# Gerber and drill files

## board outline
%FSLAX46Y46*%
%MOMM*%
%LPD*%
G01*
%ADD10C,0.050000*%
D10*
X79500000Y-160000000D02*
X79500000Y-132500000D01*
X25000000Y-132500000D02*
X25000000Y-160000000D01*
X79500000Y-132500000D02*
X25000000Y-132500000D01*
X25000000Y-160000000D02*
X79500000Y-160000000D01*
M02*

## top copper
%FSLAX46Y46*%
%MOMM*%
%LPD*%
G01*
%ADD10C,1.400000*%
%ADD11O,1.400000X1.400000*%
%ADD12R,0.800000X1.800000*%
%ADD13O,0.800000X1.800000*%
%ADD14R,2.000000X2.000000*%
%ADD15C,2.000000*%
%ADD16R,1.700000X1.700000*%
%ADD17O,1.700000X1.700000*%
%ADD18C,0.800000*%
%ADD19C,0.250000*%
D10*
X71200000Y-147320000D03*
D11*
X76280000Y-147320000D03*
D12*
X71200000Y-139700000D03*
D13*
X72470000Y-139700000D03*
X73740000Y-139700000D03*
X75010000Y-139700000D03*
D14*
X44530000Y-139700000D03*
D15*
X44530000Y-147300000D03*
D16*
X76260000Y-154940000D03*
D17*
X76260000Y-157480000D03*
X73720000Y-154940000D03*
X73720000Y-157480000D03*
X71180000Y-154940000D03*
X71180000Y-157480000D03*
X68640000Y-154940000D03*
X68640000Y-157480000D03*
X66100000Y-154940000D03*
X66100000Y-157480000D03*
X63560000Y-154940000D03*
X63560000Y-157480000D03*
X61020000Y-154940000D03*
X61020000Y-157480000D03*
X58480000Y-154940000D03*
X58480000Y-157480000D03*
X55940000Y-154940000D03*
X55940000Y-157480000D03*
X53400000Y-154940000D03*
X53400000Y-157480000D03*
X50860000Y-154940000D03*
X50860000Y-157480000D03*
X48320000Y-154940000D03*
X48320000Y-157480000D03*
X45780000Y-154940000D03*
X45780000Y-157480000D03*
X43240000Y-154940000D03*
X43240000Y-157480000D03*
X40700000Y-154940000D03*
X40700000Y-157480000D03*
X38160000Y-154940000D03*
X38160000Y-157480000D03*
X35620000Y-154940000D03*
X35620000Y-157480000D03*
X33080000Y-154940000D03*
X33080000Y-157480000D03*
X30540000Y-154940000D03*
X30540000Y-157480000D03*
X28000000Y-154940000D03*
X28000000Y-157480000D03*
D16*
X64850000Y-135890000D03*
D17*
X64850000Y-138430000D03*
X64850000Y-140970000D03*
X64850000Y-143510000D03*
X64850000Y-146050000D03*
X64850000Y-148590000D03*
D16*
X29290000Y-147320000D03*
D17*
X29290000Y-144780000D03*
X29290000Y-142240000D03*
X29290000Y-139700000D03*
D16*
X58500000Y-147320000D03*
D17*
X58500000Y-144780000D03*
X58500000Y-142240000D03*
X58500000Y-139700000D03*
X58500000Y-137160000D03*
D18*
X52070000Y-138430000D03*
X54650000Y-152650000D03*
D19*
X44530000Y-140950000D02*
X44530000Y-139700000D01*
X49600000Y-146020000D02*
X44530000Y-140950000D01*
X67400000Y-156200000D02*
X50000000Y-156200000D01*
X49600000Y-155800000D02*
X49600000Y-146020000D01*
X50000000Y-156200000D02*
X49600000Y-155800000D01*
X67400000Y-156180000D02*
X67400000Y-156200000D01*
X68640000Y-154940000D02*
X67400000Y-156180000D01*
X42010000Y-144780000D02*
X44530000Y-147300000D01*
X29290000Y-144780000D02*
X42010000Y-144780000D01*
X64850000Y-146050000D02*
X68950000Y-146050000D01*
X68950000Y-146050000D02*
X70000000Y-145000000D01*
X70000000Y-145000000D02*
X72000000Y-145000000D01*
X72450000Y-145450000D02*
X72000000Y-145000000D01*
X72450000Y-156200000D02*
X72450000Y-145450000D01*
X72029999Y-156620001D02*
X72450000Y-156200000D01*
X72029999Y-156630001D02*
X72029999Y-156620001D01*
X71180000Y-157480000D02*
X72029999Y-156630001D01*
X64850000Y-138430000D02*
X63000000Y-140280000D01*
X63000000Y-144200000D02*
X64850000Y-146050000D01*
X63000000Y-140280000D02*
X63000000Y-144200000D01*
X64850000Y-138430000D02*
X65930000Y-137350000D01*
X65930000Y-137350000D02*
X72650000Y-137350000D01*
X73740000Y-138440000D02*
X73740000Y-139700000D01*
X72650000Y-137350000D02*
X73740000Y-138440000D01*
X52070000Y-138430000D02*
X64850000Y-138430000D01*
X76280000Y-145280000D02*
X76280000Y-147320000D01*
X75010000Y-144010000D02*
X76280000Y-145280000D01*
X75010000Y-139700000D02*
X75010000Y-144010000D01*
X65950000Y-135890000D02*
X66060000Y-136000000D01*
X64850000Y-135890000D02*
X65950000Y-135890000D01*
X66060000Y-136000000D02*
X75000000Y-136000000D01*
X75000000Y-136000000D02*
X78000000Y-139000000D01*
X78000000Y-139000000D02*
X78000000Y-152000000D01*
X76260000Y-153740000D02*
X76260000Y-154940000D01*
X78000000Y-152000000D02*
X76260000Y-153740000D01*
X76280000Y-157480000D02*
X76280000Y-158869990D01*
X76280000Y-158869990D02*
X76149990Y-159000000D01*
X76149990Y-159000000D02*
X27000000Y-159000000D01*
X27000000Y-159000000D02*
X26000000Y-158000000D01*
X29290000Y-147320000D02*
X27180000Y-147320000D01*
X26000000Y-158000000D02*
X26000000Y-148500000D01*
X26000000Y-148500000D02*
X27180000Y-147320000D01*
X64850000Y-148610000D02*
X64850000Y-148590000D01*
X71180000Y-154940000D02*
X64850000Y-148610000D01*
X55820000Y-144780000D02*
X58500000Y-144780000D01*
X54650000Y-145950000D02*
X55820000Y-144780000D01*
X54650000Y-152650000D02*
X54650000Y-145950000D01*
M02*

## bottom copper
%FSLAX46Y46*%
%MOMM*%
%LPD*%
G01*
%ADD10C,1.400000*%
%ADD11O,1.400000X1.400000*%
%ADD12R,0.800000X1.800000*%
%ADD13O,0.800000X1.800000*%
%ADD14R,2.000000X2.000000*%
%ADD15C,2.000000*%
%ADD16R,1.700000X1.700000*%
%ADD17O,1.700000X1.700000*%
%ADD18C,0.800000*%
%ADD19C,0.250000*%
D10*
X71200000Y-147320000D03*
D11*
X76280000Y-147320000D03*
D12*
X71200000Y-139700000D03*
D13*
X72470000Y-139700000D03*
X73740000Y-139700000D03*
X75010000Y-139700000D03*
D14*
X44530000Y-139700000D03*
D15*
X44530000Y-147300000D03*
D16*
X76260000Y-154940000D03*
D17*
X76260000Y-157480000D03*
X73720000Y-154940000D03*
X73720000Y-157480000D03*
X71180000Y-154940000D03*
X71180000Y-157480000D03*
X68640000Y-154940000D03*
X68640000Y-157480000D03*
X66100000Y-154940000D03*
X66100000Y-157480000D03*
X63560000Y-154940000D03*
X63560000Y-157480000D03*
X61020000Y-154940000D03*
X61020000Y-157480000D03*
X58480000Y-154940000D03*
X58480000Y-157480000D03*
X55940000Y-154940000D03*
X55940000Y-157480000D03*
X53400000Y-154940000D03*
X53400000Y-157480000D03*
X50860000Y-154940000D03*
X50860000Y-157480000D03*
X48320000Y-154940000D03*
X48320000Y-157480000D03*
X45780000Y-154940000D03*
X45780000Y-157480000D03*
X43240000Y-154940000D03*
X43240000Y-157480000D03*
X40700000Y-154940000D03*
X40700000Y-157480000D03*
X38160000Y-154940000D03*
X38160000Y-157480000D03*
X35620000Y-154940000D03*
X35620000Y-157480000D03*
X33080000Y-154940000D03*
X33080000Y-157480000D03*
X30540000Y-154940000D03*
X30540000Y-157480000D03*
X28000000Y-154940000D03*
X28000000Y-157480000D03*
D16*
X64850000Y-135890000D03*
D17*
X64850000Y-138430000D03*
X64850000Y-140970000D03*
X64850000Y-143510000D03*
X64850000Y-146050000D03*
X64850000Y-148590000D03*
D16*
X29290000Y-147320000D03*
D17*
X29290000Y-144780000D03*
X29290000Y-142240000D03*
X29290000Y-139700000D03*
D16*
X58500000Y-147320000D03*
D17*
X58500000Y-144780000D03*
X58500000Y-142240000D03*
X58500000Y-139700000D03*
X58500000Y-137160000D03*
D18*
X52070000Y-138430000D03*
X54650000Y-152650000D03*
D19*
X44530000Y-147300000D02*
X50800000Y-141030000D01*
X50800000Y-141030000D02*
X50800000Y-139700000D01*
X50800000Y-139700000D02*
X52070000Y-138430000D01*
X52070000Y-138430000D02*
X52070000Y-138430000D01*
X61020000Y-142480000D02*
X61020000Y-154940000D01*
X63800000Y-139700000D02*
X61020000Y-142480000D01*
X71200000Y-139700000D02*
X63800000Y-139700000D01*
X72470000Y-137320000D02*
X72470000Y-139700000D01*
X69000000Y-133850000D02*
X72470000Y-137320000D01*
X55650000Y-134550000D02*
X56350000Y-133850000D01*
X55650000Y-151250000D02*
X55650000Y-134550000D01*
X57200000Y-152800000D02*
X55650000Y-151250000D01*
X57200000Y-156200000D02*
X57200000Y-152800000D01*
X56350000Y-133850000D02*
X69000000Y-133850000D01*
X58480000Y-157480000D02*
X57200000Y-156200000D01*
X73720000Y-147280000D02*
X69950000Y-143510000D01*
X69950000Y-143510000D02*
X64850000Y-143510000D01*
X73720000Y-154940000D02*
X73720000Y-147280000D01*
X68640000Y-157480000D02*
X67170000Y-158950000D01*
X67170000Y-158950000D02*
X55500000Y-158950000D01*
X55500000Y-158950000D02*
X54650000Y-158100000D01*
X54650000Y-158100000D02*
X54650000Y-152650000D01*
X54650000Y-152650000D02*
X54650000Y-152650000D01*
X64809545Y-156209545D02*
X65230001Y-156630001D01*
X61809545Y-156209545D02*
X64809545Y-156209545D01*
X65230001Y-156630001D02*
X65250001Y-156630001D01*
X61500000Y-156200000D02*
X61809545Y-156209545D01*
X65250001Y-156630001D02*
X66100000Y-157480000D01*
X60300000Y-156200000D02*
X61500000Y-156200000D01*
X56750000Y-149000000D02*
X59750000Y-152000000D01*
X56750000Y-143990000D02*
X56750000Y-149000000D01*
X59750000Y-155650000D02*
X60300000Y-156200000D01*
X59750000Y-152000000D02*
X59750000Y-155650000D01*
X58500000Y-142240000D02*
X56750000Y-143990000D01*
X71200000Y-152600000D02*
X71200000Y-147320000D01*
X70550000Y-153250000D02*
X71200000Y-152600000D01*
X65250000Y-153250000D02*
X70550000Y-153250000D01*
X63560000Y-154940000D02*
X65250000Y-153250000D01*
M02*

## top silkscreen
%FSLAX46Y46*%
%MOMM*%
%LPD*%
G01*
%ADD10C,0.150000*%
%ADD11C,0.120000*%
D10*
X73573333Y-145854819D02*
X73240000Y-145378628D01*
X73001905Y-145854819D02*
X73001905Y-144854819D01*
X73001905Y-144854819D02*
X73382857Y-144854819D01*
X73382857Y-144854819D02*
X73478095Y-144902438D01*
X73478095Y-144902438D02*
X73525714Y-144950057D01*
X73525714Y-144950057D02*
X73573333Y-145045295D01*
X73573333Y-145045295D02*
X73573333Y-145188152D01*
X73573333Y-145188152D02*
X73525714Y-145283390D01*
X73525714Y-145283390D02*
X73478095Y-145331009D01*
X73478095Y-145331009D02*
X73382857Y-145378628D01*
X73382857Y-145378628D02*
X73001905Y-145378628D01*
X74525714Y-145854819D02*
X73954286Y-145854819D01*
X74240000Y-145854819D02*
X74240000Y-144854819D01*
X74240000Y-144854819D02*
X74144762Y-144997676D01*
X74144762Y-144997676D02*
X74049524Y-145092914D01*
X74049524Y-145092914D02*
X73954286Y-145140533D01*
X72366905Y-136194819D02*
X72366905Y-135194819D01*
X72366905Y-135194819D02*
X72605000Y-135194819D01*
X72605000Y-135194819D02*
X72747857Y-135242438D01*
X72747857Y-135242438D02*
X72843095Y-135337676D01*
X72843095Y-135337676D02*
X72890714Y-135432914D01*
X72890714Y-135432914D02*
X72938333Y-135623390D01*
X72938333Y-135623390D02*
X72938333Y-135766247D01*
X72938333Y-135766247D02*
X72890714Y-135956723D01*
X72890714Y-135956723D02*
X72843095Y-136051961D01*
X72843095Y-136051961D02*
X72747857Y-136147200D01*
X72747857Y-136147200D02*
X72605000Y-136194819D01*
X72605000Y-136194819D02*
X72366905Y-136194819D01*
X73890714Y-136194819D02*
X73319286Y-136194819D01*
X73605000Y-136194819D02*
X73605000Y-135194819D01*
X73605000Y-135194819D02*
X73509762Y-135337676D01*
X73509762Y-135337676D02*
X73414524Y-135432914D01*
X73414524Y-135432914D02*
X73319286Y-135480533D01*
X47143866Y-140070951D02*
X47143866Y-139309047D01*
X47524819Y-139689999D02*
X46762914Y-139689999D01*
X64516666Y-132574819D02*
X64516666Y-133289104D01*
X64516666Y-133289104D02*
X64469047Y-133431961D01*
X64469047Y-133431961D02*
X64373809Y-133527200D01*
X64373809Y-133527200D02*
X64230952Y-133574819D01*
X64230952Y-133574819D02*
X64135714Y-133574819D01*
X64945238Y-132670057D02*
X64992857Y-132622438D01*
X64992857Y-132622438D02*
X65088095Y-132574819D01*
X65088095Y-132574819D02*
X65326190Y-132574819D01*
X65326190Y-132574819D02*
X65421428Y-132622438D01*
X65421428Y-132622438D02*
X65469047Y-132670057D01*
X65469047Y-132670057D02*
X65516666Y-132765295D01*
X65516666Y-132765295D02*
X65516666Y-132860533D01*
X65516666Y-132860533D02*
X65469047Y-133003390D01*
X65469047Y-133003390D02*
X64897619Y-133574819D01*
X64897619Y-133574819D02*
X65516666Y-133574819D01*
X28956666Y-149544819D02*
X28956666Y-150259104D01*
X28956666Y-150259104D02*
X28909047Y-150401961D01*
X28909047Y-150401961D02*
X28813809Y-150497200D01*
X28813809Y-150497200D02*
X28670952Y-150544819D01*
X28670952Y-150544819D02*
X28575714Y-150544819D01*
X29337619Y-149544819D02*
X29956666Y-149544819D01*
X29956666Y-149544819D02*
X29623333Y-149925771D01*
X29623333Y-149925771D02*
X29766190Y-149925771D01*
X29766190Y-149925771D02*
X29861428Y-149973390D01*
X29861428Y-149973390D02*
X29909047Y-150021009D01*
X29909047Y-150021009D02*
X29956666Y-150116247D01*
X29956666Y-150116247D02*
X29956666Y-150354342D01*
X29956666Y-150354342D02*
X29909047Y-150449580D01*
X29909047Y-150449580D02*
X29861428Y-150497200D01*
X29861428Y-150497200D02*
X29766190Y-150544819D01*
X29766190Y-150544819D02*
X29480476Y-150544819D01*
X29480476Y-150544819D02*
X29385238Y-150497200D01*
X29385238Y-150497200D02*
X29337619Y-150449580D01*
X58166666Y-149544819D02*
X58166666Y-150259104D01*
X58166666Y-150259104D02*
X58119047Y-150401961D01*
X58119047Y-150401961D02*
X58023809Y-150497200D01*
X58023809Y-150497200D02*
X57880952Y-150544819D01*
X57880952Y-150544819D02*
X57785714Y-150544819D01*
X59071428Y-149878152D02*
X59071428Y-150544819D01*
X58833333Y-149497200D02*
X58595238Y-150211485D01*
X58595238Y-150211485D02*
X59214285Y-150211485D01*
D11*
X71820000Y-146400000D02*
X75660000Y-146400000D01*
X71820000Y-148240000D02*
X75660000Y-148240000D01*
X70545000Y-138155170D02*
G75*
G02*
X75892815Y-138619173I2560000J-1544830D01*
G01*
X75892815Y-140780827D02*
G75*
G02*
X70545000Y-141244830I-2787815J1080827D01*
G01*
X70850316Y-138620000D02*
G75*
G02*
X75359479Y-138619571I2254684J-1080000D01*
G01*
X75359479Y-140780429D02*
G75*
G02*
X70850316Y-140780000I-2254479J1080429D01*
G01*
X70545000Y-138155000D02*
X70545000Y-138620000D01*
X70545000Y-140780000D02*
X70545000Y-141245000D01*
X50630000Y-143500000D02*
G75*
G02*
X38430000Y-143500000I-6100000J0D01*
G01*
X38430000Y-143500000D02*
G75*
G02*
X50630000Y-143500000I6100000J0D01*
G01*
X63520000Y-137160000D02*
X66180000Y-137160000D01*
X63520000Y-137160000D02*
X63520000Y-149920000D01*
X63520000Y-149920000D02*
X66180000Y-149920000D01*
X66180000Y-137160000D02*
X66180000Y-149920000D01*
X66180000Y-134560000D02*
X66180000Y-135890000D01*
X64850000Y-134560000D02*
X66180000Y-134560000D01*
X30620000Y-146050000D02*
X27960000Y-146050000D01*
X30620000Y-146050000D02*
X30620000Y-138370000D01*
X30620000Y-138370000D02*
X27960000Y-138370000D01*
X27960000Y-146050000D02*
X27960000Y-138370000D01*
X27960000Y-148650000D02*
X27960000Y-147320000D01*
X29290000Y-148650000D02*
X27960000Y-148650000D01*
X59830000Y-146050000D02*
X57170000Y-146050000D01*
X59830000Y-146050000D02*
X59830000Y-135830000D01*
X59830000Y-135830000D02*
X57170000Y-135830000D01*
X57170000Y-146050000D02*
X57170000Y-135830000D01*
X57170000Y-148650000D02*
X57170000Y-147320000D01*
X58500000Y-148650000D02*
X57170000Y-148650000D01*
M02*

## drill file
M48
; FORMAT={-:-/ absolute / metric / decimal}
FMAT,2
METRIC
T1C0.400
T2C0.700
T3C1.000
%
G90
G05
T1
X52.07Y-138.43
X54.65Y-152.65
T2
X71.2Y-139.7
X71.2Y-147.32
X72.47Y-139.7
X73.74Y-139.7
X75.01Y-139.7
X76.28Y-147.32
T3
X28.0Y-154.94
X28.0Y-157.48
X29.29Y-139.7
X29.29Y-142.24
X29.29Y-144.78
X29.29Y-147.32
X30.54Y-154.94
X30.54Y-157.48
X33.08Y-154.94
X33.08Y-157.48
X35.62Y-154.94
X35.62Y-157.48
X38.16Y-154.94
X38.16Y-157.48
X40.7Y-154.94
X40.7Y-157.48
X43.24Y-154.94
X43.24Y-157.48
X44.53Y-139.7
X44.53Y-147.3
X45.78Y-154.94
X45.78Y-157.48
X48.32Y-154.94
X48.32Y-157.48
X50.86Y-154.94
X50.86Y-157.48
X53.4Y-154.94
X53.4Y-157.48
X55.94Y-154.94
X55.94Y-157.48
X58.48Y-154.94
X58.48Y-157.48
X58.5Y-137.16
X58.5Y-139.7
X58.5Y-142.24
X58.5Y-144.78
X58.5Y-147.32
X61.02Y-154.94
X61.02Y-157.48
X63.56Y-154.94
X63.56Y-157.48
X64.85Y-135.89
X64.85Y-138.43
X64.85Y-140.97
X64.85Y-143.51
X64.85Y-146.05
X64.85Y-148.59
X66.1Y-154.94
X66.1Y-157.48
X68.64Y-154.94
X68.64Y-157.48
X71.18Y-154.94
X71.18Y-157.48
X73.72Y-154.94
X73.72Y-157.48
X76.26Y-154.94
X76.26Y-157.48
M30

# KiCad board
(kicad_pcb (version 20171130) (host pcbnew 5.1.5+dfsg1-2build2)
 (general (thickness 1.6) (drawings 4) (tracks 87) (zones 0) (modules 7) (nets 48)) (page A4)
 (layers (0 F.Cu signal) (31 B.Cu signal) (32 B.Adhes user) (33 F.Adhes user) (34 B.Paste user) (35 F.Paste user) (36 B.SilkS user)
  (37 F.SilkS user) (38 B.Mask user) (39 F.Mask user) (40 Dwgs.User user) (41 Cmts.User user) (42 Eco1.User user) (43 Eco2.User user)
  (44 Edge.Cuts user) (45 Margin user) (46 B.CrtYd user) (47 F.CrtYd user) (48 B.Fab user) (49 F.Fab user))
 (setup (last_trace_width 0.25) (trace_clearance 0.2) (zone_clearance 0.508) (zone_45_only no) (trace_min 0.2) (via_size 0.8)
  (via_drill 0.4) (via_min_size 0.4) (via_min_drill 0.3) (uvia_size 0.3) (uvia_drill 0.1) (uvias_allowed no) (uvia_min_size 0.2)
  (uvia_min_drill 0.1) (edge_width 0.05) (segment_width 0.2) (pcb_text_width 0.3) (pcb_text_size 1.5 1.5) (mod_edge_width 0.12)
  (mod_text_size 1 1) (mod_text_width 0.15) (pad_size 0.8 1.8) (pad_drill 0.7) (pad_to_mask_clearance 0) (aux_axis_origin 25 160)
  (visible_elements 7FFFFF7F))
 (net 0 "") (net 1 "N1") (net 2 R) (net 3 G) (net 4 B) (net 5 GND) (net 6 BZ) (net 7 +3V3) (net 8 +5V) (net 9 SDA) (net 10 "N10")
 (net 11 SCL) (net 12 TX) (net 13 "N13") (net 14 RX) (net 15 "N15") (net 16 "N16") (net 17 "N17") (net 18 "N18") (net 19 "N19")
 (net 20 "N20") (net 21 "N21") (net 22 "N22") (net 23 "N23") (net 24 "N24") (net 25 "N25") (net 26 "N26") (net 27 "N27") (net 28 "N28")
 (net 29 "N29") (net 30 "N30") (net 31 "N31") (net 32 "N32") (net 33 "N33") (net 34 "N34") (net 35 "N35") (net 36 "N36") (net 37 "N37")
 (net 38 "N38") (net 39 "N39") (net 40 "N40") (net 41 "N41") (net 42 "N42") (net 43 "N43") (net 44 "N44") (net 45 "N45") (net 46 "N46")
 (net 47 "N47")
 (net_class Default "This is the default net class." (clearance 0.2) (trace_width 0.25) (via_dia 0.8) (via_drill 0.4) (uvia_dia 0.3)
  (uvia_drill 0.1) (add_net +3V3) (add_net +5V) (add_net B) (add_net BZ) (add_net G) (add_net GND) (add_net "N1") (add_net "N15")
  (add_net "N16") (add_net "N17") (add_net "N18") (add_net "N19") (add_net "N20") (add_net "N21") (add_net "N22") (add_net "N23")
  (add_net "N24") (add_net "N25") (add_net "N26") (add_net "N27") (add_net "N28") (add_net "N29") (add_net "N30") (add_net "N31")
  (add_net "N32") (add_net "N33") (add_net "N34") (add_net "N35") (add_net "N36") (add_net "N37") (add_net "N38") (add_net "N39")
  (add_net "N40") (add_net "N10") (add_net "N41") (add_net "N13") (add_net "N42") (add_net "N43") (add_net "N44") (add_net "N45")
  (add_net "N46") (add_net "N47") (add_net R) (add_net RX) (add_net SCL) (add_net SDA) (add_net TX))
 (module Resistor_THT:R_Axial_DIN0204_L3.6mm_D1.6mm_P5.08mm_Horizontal (layer F.Cu) (at 71.2 147.32)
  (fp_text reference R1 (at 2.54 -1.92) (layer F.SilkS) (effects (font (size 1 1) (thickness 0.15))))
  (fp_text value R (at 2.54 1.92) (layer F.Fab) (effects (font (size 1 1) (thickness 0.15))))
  (fp_line (start 0.62 -0.92) (end 4.46 -0.92) (layer F.SilkS) (width 0.12))
  (fp_line (start 0.62 0.92) (end 4.46 0.92) (layer F.SilkS) (width 0.12))
  (pad 1 thru_hole circle (at 0 0) (size 1.4 1.4) (drill 0.7) (layers *.Cu *.Mask) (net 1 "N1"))
  (pad 2 thru_hole oval (at 5.08 0) (size 1.4 1.4) (drill 0.7) (layers *.Cu *.Mask) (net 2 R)))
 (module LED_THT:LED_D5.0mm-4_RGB (layer F.Cu) (at 71.2 139.7)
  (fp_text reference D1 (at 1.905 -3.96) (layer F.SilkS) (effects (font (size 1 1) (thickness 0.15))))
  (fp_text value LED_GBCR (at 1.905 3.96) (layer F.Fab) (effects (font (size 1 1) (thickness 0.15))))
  (fp_arc (start 1.905 0) (end -0.655 -1.54483) (angle 127.7) (layer F.SilkS) (width 0.12))
  (fp_arc (start 1.905 0) (end -0.655 1.54483) (angle -127.7) (layer F.SilkS) (width 0.12))
  (fp_arc (start 1.905 0) (end -0.349684 -1.08) (angle 128.8) (layer F.SilkS) (width 0.12))
  (fp_arc (start 1.905 0) (end -0.349684 1.08) (angle -128.8) (layer F.SilkS) (width 0.12))
  (fp_line (start -0.655 -1.545) (end -0.655 -1.08) (layer F.SilkS) (width 0.12))
  (fp_line (start -0.655 1.08) (end -0.655 1.545) (layer F.SilkS) (width 0.12))
  (pad 1 thru_hole rect (at 0 0) (size 0.8 1.8) (drill 0.7) (layers *.Cu *.Mask) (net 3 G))
  (pad 2 thru_hole oval (at 1.27 0) (size 0.8 1.8) (drill 0.7) (layers *.Cu *.Mask) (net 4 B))
  (pad 3 thru_hole oval (at 2.54 0) (size 0.8 1.8) (drill 0.7) (layers *.Cu *.Mask) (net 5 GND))
  (pad 4 thru_hole oval (at 3.81 0) (size 0.8 1.8) (drill 0.7) (layers *.Cu *.Mask) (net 2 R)))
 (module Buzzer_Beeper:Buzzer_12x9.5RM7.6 (layer F.Cu) (at 44.53 139.7 270)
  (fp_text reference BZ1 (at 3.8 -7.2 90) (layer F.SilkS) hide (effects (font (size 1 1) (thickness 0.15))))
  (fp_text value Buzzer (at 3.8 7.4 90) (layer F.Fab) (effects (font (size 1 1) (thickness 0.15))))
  (fp_circle (center 3.8 0) (end 9.9 0) (layer F.SilkS) (width 0.12))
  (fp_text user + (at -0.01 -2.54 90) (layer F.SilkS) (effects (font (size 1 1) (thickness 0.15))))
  (pad 1 thru_hole rect (at 0 0 270) (size 2 2) (drill 1) (layers *.Cu *.Mask) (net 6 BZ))
  (pad 2 thru_hole circle (at 7.6 0 270) (size 2 2) (drill 1) (layers *.Cu *.Mask) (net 5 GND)))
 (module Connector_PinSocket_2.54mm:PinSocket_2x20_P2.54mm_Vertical (layer B.Cu) (at 76.26 154.94 90)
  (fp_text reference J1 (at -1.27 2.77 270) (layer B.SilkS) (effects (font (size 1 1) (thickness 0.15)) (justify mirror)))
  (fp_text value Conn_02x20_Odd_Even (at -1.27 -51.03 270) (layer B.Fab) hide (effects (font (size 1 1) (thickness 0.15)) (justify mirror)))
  (pad 1 thru_hole rect (at 0 0 90) (size 1.7 1.7) (drill 1) (layers *.Cu *.Mask) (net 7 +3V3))
  (pad 2 thru_hole oval (at -2.54 0 90) (size 1.7 1.7) (drill 1) (layers *.Cu *.Mask) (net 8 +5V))
  (pad 3 thru_hole oval (at 0 -2.54 90) (size 1.7 1.7) (drill 1) (layers *.Cu *.Mask) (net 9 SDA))
  (pad 4 thru_hole oval (at -2.54 -2.54 90) (size 1.7 1.7) (drill 1) (layers *.Cu *.Mask) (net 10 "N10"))
  (pad 5 thru_hole oval (at 0 -5.08 90) (size 1.7 1.7) (drill 1) (layers *.Cu *.Mask) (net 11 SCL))
  (pad 6 thru_hole oval (at -2.54 -5.08 90) (size 1.7 1.7) (drill 1) (layers *.Cu *.Mask) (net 5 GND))
  (pad 7 thru_hole oval (at 0 -7.62 90) (size 1.7 1.7) (drill 1) (layers *.Cu *.Mask) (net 6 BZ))
  (pad 8 thru_hole oval (at -2.54 -7.62 90) (size 1.7 1.7) (drill 1) (layers *.Cu *.Mask) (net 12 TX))
  (pad 9 thru_hole oval (at 0 -10.16 90) (size 1.7 1.7) (drill 1) (layers *.Cu *.Mask) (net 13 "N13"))
  (pad 10 thru_hole oval (at -2.54 -10.16 90) (size 1.7 1.7) (drill 1) (layers *.Cu *.Mask) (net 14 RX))
  (pad 11 thru_hole oval (at 0 -12.7 90) (size 1.7 1.7) (drill 1) (layers *.Cu *.Mask) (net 1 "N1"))
  (pad 12 thru_hole oval (at -2.54 -12.7 90) (size 1.7 1.7) (drill 1) (layers *.Cu *.Mask) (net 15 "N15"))
  (pad 13 thru_hole oval (at 0 -15.24 90) (size 1.7 1.7) (drill 1) (layers *.Cu *.Mask) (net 3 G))
  (pad 14 thru_hole oval (at -2.54 -15.24 90) (size 1.7 1.7) (drill 1) (layers *.Cu *.Mask) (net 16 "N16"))
  (pad 15 thru_hole oval (at 0 -17.78 90) (size 1.7 1.7) (drill 1) (layers *.Cu *.Mask) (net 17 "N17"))
  (pad 16 thru_hole oval (at -2.54 -17.78 90) (size 1.7 1.7) (drill 1) (layers *.Cu *.Mask) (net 4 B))
  (pad 17 thru_hole oval (at 0 -20.32 90) (size 1.7 1.7) (drill 1) (layers *.Cu *.Mask) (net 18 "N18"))
  (pad 18 thru_hole oval (at -2.54 -20.32 90) (size 1.7 1.7) (drill 1) (layers *.Cu *.Mask) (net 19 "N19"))
  (pad 19 thru_hole oval (at 0 -22.86 90) (size 1.7 1.7) (drill 1) (layers *.Cu *.Mask) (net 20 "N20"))
  (pad 20 thru_hole oval (at -2.54 -22.86 90) (size 1.7 1.7) (drill 1) (layers *.Cu *.Mask) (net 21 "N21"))
  (pad 21 thru_hole oval (at 0 -25.4 90) (size 1.7 1.7) (drill 1) (layers *.Cu *.Mask) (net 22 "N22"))
  (pad 22 thru_hole oval (at -2.54 -25.4 90) (size 1.7 1.7) (drill 1) (layers *.Cu *.Mask) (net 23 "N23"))
  (pad 23 thru_hole oval (at 0 -27.94 90) (size 1.7 1.7) (drill 1) (layers *.Cu *.Mask) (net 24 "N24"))
  (pad 24 thru_hole oval (at -2.54 -27.94 90) (size 1.7 1.7) (drill 1) (layers *.Cu *.Mask) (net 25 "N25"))
  (pad 25 thru_hole oval (at 0 -30.48 90) (size 1.7 1.7) (drill 1) (layers *.Cu *.Mask) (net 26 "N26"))
  (pad 26 thru_hole oval (at -2.54 -30.48 90) (size 1.7 1.7) (drill 1) (layers *.Cu *.Mask) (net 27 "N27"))
  (pad 27 thru_hole oval (at 0 -33.02 90) (size 1.7 1.7) (drill 1) (layers *.Cu *.Mask) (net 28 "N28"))
  (pad 28 thru_hole oval (at -2.54 -33.02 90) (size 1.7 1.7) (drill 1) (layers *.Cu *.Mask) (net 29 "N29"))
  (pad 29 thru_hole oval (at 0 -35.56 90) (size 1.7 1.7) (drill 1) (layers *.Cu *.Mask) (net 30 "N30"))
  (pad 30 thru_hole oval (at -2.54 -35.56 90) (size 1.7 1.7) (drill 1) (layers *.Cu *.Mask) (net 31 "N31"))
  (pad 31 thru_hole oval (at 0 -38.1 90) (size 1.7 1.7) (drill 1) (layers *.Cu *.Mask) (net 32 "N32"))
  (pad 32 thru_hole oval (at -2.54 -38.1 90) (size 1.7 1.7) (drill 1) (layers *.Cu *.Mask) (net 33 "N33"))
  (pad 33 thru_hole oval (at 0 -40.64 90) (size 1.7 1.7) (drill 1) (layers *.Cu *.Mask) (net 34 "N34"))
  (pad 34 thru_hole oval (at -2.54 -40.64 90) (size 1.7 1.7) (drill 1) (layers *.Cu *.Mask) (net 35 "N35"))
  (pad 35 thru_hole oval (at 0 -43.18 90) (size 1.7 1.7) (drill 1) (layers *.Cu *.Mask) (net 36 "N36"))
  (pad 36 thru_hole oval (at -2.54 -43.18 90) (size 1.7 1.7) (drill 1) (layers *.Cu *.Mask) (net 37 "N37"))
  (pad 37 thru_hole oval (at 0 -45.72 90) (size 1.7 1.7) (drill 1) (layers *.Cu *.Mask) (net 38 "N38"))
  (pad 38 thru_hole oval (at -2.54 -45.72 90) (size 1.7 1.7) (drill 1) (layers *.Cu *.Mask) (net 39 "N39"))
  (pad 39 thru_hole oval (at 0 -48.26 90) (size 1.7 1.7) (drill 1) (layers *.Cu *.Mask) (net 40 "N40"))
  (pad 40 thru_hole oval (at -2.54 -48.26 90) (size 1.7 1.7) (drill 1) (layers *.Cu *.Mask) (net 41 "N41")))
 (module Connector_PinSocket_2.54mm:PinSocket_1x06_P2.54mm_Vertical (layer F.Cu) (at 64.85 135.89)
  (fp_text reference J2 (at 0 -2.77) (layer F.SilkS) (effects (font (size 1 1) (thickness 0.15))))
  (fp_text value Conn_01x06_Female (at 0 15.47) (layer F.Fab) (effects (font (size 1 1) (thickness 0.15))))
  (fp_line (start -1.33 1.27) (end 1.33 1.27) (layer F.SilkS) (width 0.12))
  (fp_line (start -1.33 1.27) (end -1.33 14.03) (layer F.SilkS) (width 0.12))
  (fp_line (start -1.33 14.03) (end 1.33 14.03) (layer F.SilkS) (width 0.12))
  (fp_line (start 1.33 1.27) (end 1.33 14.03) (layer F.SilkS) (width 0.12))
  (fp_line (start 1.33 -1.33) (end 1.33 0) (layer F.SilkS) (width 0.12))
  (fp_line (start 0 -1.33) (end 1.33 -1.33) (layer F.SilkS) (width 0.12))
  (pad 1 thru_hole rect (at 0 0) (size 1.7 1.7) (drill 1) (layers *.Cu *.Mask) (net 7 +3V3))
  (pad 2 thru_hole oval (at 0 2.54) (size 1.7 1.7) (drill 1) (layers *.Cu *.Mask) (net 5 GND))
  (pad 3 thru_hole oval (at 0 5.08) (size 1.7 1.7) (drill 1) (layers *.Cu *.Mask) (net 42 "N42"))
  (pad 4 thru_hole oval (at 0 7.62) (size 1.7 1.7) (drill 1) (layers *.Cu *.Mask) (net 9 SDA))
  (pad 5 thru_hole oval (at 0 10.16) (size 1.7 1.7) (drill 1) (layers *.Cu *.Mask) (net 5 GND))
  (pad 6 thru_hole oval (at 0 12.7) (size 1.7 1.7) (drill 1) (layers *.Cu *.Mask) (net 11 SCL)))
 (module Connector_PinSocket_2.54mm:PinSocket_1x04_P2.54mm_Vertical (layer F.Cu) (at 29.29 147.32 180)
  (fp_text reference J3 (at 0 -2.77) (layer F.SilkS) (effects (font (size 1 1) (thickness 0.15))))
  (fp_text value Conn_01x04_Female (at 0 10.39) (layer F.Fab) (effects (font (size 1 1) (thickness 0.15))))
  (fp_line (start -1.33 1.27) (end 1.33 1.27) (layer F.SilkS) (width 0.12))
  (fp_line (start -1.33 1.27) (end -1.33 8.95) (layer F.SilkS) (width 0.12))
  (fp_line (start -1.33 8.95) (end 1.33 8.95) (layer F.SilkS) (width 0.12))
  (fp_line (start 1.33 1.27) (end 1.33 8.95) (layer F.SilkS) (width 0.12))
  (fp_line (start 1.33 -1.33) (end 1.33 0) (layer F.SilkS) (width 0.12))
  (fp_line (start 0 -1.33) (end 1.33 -1.33) (layer F.SilkS) (width 0.12))
  (pad 1 thru_hole rect (at 0 0 180) (size 1.7 1.7) (drill 1) (layers *.Cu *.Mask) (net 8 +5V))
  (pad 2 thru_hole oval (at 0 2.54 180) (size 1.7 1.7) (drill 1) (layers *.Cu *.Mask) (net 5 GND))
  (pad 3 thru_hole oval (at 0 5.08 180) (size 1.7 1.7) (drill 1) (layers *.Cu *.Mask) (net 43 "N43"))
  (pad 4 thru_hole oval (at 0 7.62 180) (size 1.7 1.7) (drill 1) (layers *.Cu *.Mask) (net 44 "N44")))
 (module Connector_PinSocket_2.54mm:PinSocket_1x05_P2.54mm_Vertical (layer F.Cu) (at 58.5 147.32 180)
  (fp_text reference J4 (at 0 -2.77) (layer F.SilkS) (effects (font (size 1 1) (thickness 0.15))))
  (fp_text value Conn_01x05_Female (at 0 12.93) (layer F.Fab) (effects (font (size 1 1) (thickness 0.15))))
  (fp_line (start -1.33 1.27) (end 1.33 1.27) (layer F.SilkS) (width 0.12))
  (fp_line (start -1.33 1.27) (end -1.33 11.49) (layer F.SilkS) (width 0.12))
  (fp_line (start -1.33 11.49) (end 1.33 11.49) (layer F.SilkS) (width 0.12))
  (fp_line (start 1.33 1.27) (end 1.33 11.49) (layer F.SilkS) (width 0.12))
  (fp_line (start 1.33 -1.33) (end 1.33 0) (layer F.SilkS) (width 0.12))
  (fp_line (start 0 -1.33) (end 1.33 -1.33) (layer F.SilkS) (width 0.12))
  (pad 1 thru_hole rect (at 0 0 180) (size 1.7 1.7) (drill 1) (layers *.Cu *.Mask) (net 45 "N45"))
  (pad 2 thru_hole oval (at 0 2.54 180) (size 1.7 1.7) (drill 1) (layers *.Cu *.Mask) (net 12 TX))
  (pad 3 thru_hole oval (at 0 5.08 180) (size 1.7 1.7) (drill 1) (layers *.Cu *.Mask) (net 14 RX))
  (pad 4 thru_hole oval (at 0 7.62 180) (size 1.7 1.7) (drill 1) (layers *.Cu *.Mask) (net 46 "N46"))
  (pad 5 thru_hole oval (at 0 10.16 180) (size 1.7 1.7) (drill 1) (layers *.Cu *.Mask) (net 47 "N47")))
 (gr_line (start 79.5 160) (end 79.5 132.5) (layer Edge.Cuts) (width 0.05))
 (gr_line (start 25 132.5) (end 25 160) (layer Edge.Cuts) (width 0.05))
 (gr_line (start 79.5 132.5) (end 25 132.5) (layer Edge.Cuts) (width 0.05))
 (gr_line (start 25 160) (end 79.5 160) (layer Edge.Cuts) (width 0.05))
 (segment (start 44.53 140.95) (end 44.53 139.7) (width 0.25) (layer F.Cu) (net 6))
 (segment (start 49.6 146.02) (end 44.53 140.95) (width 0.25) (layer F.Cu) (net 6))
 (segment (start 67.4 156.2) (end 50 156.2) (width 0.25) (layer F.Cu) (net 6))
 (segment (start 49.6 155.8) (end 49.6 146.02) (width 0.25) (layer F.Cu) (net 6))
 (segment (start 50 156.2) (end 49.6 155.8) (width 0.25) (layer F.Cu) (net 6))
 (segment (start 67.4 156.18) (end 67.4 156.2) (width 0.25) (layer F.Cu) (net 6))
 (segment (start 68.64 154.94) (end 67.4 156.18) (width 0.25) (layer F.Cu) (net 6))
 (segment (start 42.01 144.78) (end 44.53 147.3) (width 0.25) (layer F.Cu) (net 5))
 (segment (start 29.29 144.78) (end 42.01 144.78) (width 0.25) (layer F.Cu) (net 5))
 (segment (start 64.85 146.05) (end 68.95 146.05) (width 0.25) (layer F.Cu) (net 5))
 (segment (start 68.95 146.05) (end 70 145) (width 0.25) (layer F.Cu) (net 5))
 (segment (start 70 145) (end 72 145) (width 0.25) (layer F.Cu) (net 5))
 (segment (start 72.45 145.45) (end 72 145) (width 0.25) (layer F.Cu) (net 5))
 (segment (start 72.45 156.2) (end 72.45 145.45) (width 0.25) (layer F.Cu) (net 5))
 (segment (start 72.029999 156.620001) (end 72.45 156.2) (width 0.25) (layer F.Cu) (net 5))
 (segment (start 72.029999 156.630001) (end 72.029999 156.620001) (width 0.25) (layer F.Cu) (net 5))
 (segment (start 71.18 157.48) (end 72.029999 156.630001) (width 0.25) (layer F.Cu) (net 5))
 (segment (start 64.85 138.43) (end 63 140.28) (width 0.25) (layer F.Cu) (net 5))
 (segment (start 63 144.2) (end 64.85 146.05) (width 0.25) (layer F.Cu) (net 5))
 (segment (start 63 140.28) (end 63 144.2) (width 0.25) (layer F.Cu) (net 5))
 (segment (start 64.85 138.43) (end 65.93 137.35) (width 0.25) (layer F.Cu) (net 5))
 (segment (start 65.93 137.35) (end 72.65 137.35) (width 0.25) (layer F.Cu) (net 5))
 (segment (start 73.74 138.44) (end 73.74 139.7) (width 0.25) (layer F.Cu) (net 5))
 (segment (start 72.65 137.35) (end 73.74 138.44) (width 0.25) (layer F.Cu) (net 5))
 (segment (start 44.53 147.3) (end 50.8 141.03) (width 0.25) (layer B.Cu) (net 5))
 (segment (start 50.8 141.03) (end 50.8 139.7) (width 0.25) (layer B.Cu) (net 5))
 (segment (start 50.8 139.7) (end 52.07 138.43) (width 0.25) (layer B.Cu) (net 5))
 (segment (start 52.07 138.43) (end 52.07 138.43) (width 0.25) (layer B.Cu) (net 5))
 (via (at 52.07 138.43) (size 0.8) (drill 0.4) (layers F.Cu B.Cu) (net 5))
 (segment (start 52.07 138.43) (end 64.85 138.43) (width 0.25) (layer F.Cu) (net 5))
 (segment (start 61.02 142.48) (end 61.02 154.94) (width 0.25) (layer B.Cu) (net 3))
 (segment (start 63.8 139.7) (end 61.02 142.48) (width 0.25) (layer B.Cu) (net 3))
 (segment (start 71.2 139.7) (end 63.8 139.7) (width 0.25) (layer B.Cu) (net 3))
 (segment (start 72.47 137.32) (end 72.47 139.7) (width 0.25) (layer B.Cu) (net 4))
 (segment (start 69 133.85) (end 72.47 137.32) (width 0.25) (layer B.Cu) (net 4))
 (segment (start 55.65 134.55) (end 56.35 133.85) (width 0.25) (layer B.Cu) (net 4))
 (segment (start 55.65 151.25) (end 55.65 134.55) (width 0.25) (layer B.Cu) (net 4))
 (segment (start 57.2 152.8) (end 55.65 151.25) (width 0.25) (layer B.Cu) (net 4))
 (segment (start 57.2 156.2) (end 57.2 152.8) (width 0.25) (layer B.Cu) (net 4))
 (segment (start 56.35 133.85) (end 69 133.85) (width 0.25) (layer B.Cu) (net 4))
 (segment (start 58.48 157.48) (end 57.2 156.2) (width 0.25) (layer B.Cu) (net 4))
 (segment (start 76.28 145.28) (end 76.28 147.32) (width 0.25) (layer F.Cu) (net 2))
 (segment (start 75.01 144.01) (end 76.28 145.28) (width 0.25) (layer F.Cu) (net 2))
 (segment (start 75.01 139.7) (end 75.01 144.01) (width 0.25) (layer F.Cu) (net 2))
 (segment (start 65.95 135.89) (end 66.06 136) (width 0.25) (layer F.Cu) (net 7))
 (segment (start 64.85 135.89) (end 65.95 135.89) (width 0.25) (layer F.Cu) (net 7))
 (segment (start 66.06 136) (end 75 136) (width 0.25) (layer F.Cu) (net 7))
 (segment (start 75 136) (end 78 139) (width 0.25) (layer F.Cu) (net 7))
 (segment (start 78 139) (end 78 152) (width 0.25) (layer F.Cu) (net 7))
 (segment (start 76.26 153.74) (end 76.26 154.94) (width 0.25) (layer F.Cu) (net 7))
 (segment (start 78 152) (end 76.26 153.74) (width 0.25) (layer F.Cu) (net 7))
 (segment (start 76.28 157.48) (end 76.28 158.86999) (width 0.25) (layer F.Cu) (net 8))
 (segment (start 76.28 158.86999) (end 76.14999 159) (width 0.25) (layer F.Cu) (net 8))
 (segment (start 76.14999 159) (end 27 159) (width 0.25) (layer F.Cu) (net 8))
 (segment (start 27 159) (end 26 158) (width 0.25) (layer F.Cu) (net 8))
 (segment (start 29.29 147.32) (end 27.18 147.32) (width 0.25) (layer F.Cu) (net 8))
 (segment (start 26 158) (end 26 148.5) (width 0.25) (layer F.Cu) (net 8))
 (segment (start 26 148.5) (end 27.18 147.32) (width 0.25) (layer F.Cu) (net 8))
 (segment (start 73.72 147.28) (end 69.95 143.51) (width 0.25) (layer B.Cu) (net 9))
 (segment (start 69.95 143.51) (end 64.85 143.51) (width 0.25) (layer B.Cu) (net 9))
 (segment (start 73.72 154.94) (end 73.72 147.28) (width 0.25) (layer B.Cu) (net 9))
 (segment (start 64.85 148.61) (end 64.85 148.59) (width 0.25) (layer F.Cu) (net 11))
 (segment (start 71.18 154.94) (end 64.85 148.61) (width 0.25) (layer F.Cu) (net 11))
 (segment (start 68.64 157.48) (end 67.17 158.95) (width 0.25) (layer B.Cu) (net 12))
 (segment (start 67.17 158.95) (end 55.5 158.95) (width 0.25) (layer B.Cu) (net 12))
 (segment (start 55.5 158.95) (end 54.65 158.1) (width 0.25) (layer B.Cu) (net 12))
 (segment (start 54.65 158.1) (end 54.65 152.65) (width 0.25) (layer B.Cu) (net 12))
 (segment (start 54.65 152.65) (end 54.65 152.65) (width 0.25) (layer B.Cu) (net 12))
 (via (at 54.65 152.65) (size 0.8) (drill 0.4) (layers F.Cu B.Cu) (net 12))
 (segment (start 55.82 144.78) (end 58.5 144.78) (width 0.25) (layer F.Cu) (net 12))
 (segment (start 54.65 145.95) (end 55.82 144.78) (width 0.25) (layer F.Cu) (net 12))
 (segment (start 54.65 152.65) (end 54.65 145.95) (width 0.25) (layer F.Cu) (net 12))
 (segment (start 64.809545 156.209545) (end 65.230001 156.630001) (width 0.25) (layer B.Cu) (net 14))
 (segment (start 61.809545 156.209545) (end 64.809545 156.209545) (width 0.25) (layer B.Cu) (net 14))
 (segment (start 65.230001 156.630001) (end 65.250001 156.630001) (width 0.25) (layer B.Cu) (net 14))
 (segment (start 61.5 156.2) (end 61.809545 156.209545) (width 0.25) (layer B.Cu) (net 14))
 (segment (start 65.250001 156.630001) (end 66.1 157.48) (width 0.25) (layer B.Cu) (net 14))
 (segment (start 60.3 156.2) (end 61.5 156.2) (width 0.25) (layer B.Cu) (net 14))
 (segment (start 56.75 149) (end 59.75 152) (width 0.25) (layer B.Cu) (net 14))
 (segment (start 56.75 143.99) (end 56.75 149) (width 0.25) (layer B.Cu) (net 14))
 (segment (start 59.75 155.65) (end 60.3 156.2) (width 0.25) (layer B.Cu) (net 14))
 (segment (start 59.75 152) (end 59.75 155.65) (width 0.25) (layer B.Cu) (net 14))
 (segment (start 58.5 142.24) (end 56.75 143.99) (width 0.25) (layer B.Cu) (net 14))
 (segment (start 71.2 152.6) (end 71.2 147.32) (width 0.25) (layer B.Cu) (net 1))
 (segment (start 70.55 153.25) (end 71.2 152.6) (width 0.25) (layer B.Cu) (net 1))
 (segment (start 65.25 153.25) (end 70.55 153.25) (width 0.25) (layer B.Cu) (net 1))
 (segment (start 63.56 154.94) (end 65.25 153.25) (width 0.25) (layer B.Cu) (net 1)))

